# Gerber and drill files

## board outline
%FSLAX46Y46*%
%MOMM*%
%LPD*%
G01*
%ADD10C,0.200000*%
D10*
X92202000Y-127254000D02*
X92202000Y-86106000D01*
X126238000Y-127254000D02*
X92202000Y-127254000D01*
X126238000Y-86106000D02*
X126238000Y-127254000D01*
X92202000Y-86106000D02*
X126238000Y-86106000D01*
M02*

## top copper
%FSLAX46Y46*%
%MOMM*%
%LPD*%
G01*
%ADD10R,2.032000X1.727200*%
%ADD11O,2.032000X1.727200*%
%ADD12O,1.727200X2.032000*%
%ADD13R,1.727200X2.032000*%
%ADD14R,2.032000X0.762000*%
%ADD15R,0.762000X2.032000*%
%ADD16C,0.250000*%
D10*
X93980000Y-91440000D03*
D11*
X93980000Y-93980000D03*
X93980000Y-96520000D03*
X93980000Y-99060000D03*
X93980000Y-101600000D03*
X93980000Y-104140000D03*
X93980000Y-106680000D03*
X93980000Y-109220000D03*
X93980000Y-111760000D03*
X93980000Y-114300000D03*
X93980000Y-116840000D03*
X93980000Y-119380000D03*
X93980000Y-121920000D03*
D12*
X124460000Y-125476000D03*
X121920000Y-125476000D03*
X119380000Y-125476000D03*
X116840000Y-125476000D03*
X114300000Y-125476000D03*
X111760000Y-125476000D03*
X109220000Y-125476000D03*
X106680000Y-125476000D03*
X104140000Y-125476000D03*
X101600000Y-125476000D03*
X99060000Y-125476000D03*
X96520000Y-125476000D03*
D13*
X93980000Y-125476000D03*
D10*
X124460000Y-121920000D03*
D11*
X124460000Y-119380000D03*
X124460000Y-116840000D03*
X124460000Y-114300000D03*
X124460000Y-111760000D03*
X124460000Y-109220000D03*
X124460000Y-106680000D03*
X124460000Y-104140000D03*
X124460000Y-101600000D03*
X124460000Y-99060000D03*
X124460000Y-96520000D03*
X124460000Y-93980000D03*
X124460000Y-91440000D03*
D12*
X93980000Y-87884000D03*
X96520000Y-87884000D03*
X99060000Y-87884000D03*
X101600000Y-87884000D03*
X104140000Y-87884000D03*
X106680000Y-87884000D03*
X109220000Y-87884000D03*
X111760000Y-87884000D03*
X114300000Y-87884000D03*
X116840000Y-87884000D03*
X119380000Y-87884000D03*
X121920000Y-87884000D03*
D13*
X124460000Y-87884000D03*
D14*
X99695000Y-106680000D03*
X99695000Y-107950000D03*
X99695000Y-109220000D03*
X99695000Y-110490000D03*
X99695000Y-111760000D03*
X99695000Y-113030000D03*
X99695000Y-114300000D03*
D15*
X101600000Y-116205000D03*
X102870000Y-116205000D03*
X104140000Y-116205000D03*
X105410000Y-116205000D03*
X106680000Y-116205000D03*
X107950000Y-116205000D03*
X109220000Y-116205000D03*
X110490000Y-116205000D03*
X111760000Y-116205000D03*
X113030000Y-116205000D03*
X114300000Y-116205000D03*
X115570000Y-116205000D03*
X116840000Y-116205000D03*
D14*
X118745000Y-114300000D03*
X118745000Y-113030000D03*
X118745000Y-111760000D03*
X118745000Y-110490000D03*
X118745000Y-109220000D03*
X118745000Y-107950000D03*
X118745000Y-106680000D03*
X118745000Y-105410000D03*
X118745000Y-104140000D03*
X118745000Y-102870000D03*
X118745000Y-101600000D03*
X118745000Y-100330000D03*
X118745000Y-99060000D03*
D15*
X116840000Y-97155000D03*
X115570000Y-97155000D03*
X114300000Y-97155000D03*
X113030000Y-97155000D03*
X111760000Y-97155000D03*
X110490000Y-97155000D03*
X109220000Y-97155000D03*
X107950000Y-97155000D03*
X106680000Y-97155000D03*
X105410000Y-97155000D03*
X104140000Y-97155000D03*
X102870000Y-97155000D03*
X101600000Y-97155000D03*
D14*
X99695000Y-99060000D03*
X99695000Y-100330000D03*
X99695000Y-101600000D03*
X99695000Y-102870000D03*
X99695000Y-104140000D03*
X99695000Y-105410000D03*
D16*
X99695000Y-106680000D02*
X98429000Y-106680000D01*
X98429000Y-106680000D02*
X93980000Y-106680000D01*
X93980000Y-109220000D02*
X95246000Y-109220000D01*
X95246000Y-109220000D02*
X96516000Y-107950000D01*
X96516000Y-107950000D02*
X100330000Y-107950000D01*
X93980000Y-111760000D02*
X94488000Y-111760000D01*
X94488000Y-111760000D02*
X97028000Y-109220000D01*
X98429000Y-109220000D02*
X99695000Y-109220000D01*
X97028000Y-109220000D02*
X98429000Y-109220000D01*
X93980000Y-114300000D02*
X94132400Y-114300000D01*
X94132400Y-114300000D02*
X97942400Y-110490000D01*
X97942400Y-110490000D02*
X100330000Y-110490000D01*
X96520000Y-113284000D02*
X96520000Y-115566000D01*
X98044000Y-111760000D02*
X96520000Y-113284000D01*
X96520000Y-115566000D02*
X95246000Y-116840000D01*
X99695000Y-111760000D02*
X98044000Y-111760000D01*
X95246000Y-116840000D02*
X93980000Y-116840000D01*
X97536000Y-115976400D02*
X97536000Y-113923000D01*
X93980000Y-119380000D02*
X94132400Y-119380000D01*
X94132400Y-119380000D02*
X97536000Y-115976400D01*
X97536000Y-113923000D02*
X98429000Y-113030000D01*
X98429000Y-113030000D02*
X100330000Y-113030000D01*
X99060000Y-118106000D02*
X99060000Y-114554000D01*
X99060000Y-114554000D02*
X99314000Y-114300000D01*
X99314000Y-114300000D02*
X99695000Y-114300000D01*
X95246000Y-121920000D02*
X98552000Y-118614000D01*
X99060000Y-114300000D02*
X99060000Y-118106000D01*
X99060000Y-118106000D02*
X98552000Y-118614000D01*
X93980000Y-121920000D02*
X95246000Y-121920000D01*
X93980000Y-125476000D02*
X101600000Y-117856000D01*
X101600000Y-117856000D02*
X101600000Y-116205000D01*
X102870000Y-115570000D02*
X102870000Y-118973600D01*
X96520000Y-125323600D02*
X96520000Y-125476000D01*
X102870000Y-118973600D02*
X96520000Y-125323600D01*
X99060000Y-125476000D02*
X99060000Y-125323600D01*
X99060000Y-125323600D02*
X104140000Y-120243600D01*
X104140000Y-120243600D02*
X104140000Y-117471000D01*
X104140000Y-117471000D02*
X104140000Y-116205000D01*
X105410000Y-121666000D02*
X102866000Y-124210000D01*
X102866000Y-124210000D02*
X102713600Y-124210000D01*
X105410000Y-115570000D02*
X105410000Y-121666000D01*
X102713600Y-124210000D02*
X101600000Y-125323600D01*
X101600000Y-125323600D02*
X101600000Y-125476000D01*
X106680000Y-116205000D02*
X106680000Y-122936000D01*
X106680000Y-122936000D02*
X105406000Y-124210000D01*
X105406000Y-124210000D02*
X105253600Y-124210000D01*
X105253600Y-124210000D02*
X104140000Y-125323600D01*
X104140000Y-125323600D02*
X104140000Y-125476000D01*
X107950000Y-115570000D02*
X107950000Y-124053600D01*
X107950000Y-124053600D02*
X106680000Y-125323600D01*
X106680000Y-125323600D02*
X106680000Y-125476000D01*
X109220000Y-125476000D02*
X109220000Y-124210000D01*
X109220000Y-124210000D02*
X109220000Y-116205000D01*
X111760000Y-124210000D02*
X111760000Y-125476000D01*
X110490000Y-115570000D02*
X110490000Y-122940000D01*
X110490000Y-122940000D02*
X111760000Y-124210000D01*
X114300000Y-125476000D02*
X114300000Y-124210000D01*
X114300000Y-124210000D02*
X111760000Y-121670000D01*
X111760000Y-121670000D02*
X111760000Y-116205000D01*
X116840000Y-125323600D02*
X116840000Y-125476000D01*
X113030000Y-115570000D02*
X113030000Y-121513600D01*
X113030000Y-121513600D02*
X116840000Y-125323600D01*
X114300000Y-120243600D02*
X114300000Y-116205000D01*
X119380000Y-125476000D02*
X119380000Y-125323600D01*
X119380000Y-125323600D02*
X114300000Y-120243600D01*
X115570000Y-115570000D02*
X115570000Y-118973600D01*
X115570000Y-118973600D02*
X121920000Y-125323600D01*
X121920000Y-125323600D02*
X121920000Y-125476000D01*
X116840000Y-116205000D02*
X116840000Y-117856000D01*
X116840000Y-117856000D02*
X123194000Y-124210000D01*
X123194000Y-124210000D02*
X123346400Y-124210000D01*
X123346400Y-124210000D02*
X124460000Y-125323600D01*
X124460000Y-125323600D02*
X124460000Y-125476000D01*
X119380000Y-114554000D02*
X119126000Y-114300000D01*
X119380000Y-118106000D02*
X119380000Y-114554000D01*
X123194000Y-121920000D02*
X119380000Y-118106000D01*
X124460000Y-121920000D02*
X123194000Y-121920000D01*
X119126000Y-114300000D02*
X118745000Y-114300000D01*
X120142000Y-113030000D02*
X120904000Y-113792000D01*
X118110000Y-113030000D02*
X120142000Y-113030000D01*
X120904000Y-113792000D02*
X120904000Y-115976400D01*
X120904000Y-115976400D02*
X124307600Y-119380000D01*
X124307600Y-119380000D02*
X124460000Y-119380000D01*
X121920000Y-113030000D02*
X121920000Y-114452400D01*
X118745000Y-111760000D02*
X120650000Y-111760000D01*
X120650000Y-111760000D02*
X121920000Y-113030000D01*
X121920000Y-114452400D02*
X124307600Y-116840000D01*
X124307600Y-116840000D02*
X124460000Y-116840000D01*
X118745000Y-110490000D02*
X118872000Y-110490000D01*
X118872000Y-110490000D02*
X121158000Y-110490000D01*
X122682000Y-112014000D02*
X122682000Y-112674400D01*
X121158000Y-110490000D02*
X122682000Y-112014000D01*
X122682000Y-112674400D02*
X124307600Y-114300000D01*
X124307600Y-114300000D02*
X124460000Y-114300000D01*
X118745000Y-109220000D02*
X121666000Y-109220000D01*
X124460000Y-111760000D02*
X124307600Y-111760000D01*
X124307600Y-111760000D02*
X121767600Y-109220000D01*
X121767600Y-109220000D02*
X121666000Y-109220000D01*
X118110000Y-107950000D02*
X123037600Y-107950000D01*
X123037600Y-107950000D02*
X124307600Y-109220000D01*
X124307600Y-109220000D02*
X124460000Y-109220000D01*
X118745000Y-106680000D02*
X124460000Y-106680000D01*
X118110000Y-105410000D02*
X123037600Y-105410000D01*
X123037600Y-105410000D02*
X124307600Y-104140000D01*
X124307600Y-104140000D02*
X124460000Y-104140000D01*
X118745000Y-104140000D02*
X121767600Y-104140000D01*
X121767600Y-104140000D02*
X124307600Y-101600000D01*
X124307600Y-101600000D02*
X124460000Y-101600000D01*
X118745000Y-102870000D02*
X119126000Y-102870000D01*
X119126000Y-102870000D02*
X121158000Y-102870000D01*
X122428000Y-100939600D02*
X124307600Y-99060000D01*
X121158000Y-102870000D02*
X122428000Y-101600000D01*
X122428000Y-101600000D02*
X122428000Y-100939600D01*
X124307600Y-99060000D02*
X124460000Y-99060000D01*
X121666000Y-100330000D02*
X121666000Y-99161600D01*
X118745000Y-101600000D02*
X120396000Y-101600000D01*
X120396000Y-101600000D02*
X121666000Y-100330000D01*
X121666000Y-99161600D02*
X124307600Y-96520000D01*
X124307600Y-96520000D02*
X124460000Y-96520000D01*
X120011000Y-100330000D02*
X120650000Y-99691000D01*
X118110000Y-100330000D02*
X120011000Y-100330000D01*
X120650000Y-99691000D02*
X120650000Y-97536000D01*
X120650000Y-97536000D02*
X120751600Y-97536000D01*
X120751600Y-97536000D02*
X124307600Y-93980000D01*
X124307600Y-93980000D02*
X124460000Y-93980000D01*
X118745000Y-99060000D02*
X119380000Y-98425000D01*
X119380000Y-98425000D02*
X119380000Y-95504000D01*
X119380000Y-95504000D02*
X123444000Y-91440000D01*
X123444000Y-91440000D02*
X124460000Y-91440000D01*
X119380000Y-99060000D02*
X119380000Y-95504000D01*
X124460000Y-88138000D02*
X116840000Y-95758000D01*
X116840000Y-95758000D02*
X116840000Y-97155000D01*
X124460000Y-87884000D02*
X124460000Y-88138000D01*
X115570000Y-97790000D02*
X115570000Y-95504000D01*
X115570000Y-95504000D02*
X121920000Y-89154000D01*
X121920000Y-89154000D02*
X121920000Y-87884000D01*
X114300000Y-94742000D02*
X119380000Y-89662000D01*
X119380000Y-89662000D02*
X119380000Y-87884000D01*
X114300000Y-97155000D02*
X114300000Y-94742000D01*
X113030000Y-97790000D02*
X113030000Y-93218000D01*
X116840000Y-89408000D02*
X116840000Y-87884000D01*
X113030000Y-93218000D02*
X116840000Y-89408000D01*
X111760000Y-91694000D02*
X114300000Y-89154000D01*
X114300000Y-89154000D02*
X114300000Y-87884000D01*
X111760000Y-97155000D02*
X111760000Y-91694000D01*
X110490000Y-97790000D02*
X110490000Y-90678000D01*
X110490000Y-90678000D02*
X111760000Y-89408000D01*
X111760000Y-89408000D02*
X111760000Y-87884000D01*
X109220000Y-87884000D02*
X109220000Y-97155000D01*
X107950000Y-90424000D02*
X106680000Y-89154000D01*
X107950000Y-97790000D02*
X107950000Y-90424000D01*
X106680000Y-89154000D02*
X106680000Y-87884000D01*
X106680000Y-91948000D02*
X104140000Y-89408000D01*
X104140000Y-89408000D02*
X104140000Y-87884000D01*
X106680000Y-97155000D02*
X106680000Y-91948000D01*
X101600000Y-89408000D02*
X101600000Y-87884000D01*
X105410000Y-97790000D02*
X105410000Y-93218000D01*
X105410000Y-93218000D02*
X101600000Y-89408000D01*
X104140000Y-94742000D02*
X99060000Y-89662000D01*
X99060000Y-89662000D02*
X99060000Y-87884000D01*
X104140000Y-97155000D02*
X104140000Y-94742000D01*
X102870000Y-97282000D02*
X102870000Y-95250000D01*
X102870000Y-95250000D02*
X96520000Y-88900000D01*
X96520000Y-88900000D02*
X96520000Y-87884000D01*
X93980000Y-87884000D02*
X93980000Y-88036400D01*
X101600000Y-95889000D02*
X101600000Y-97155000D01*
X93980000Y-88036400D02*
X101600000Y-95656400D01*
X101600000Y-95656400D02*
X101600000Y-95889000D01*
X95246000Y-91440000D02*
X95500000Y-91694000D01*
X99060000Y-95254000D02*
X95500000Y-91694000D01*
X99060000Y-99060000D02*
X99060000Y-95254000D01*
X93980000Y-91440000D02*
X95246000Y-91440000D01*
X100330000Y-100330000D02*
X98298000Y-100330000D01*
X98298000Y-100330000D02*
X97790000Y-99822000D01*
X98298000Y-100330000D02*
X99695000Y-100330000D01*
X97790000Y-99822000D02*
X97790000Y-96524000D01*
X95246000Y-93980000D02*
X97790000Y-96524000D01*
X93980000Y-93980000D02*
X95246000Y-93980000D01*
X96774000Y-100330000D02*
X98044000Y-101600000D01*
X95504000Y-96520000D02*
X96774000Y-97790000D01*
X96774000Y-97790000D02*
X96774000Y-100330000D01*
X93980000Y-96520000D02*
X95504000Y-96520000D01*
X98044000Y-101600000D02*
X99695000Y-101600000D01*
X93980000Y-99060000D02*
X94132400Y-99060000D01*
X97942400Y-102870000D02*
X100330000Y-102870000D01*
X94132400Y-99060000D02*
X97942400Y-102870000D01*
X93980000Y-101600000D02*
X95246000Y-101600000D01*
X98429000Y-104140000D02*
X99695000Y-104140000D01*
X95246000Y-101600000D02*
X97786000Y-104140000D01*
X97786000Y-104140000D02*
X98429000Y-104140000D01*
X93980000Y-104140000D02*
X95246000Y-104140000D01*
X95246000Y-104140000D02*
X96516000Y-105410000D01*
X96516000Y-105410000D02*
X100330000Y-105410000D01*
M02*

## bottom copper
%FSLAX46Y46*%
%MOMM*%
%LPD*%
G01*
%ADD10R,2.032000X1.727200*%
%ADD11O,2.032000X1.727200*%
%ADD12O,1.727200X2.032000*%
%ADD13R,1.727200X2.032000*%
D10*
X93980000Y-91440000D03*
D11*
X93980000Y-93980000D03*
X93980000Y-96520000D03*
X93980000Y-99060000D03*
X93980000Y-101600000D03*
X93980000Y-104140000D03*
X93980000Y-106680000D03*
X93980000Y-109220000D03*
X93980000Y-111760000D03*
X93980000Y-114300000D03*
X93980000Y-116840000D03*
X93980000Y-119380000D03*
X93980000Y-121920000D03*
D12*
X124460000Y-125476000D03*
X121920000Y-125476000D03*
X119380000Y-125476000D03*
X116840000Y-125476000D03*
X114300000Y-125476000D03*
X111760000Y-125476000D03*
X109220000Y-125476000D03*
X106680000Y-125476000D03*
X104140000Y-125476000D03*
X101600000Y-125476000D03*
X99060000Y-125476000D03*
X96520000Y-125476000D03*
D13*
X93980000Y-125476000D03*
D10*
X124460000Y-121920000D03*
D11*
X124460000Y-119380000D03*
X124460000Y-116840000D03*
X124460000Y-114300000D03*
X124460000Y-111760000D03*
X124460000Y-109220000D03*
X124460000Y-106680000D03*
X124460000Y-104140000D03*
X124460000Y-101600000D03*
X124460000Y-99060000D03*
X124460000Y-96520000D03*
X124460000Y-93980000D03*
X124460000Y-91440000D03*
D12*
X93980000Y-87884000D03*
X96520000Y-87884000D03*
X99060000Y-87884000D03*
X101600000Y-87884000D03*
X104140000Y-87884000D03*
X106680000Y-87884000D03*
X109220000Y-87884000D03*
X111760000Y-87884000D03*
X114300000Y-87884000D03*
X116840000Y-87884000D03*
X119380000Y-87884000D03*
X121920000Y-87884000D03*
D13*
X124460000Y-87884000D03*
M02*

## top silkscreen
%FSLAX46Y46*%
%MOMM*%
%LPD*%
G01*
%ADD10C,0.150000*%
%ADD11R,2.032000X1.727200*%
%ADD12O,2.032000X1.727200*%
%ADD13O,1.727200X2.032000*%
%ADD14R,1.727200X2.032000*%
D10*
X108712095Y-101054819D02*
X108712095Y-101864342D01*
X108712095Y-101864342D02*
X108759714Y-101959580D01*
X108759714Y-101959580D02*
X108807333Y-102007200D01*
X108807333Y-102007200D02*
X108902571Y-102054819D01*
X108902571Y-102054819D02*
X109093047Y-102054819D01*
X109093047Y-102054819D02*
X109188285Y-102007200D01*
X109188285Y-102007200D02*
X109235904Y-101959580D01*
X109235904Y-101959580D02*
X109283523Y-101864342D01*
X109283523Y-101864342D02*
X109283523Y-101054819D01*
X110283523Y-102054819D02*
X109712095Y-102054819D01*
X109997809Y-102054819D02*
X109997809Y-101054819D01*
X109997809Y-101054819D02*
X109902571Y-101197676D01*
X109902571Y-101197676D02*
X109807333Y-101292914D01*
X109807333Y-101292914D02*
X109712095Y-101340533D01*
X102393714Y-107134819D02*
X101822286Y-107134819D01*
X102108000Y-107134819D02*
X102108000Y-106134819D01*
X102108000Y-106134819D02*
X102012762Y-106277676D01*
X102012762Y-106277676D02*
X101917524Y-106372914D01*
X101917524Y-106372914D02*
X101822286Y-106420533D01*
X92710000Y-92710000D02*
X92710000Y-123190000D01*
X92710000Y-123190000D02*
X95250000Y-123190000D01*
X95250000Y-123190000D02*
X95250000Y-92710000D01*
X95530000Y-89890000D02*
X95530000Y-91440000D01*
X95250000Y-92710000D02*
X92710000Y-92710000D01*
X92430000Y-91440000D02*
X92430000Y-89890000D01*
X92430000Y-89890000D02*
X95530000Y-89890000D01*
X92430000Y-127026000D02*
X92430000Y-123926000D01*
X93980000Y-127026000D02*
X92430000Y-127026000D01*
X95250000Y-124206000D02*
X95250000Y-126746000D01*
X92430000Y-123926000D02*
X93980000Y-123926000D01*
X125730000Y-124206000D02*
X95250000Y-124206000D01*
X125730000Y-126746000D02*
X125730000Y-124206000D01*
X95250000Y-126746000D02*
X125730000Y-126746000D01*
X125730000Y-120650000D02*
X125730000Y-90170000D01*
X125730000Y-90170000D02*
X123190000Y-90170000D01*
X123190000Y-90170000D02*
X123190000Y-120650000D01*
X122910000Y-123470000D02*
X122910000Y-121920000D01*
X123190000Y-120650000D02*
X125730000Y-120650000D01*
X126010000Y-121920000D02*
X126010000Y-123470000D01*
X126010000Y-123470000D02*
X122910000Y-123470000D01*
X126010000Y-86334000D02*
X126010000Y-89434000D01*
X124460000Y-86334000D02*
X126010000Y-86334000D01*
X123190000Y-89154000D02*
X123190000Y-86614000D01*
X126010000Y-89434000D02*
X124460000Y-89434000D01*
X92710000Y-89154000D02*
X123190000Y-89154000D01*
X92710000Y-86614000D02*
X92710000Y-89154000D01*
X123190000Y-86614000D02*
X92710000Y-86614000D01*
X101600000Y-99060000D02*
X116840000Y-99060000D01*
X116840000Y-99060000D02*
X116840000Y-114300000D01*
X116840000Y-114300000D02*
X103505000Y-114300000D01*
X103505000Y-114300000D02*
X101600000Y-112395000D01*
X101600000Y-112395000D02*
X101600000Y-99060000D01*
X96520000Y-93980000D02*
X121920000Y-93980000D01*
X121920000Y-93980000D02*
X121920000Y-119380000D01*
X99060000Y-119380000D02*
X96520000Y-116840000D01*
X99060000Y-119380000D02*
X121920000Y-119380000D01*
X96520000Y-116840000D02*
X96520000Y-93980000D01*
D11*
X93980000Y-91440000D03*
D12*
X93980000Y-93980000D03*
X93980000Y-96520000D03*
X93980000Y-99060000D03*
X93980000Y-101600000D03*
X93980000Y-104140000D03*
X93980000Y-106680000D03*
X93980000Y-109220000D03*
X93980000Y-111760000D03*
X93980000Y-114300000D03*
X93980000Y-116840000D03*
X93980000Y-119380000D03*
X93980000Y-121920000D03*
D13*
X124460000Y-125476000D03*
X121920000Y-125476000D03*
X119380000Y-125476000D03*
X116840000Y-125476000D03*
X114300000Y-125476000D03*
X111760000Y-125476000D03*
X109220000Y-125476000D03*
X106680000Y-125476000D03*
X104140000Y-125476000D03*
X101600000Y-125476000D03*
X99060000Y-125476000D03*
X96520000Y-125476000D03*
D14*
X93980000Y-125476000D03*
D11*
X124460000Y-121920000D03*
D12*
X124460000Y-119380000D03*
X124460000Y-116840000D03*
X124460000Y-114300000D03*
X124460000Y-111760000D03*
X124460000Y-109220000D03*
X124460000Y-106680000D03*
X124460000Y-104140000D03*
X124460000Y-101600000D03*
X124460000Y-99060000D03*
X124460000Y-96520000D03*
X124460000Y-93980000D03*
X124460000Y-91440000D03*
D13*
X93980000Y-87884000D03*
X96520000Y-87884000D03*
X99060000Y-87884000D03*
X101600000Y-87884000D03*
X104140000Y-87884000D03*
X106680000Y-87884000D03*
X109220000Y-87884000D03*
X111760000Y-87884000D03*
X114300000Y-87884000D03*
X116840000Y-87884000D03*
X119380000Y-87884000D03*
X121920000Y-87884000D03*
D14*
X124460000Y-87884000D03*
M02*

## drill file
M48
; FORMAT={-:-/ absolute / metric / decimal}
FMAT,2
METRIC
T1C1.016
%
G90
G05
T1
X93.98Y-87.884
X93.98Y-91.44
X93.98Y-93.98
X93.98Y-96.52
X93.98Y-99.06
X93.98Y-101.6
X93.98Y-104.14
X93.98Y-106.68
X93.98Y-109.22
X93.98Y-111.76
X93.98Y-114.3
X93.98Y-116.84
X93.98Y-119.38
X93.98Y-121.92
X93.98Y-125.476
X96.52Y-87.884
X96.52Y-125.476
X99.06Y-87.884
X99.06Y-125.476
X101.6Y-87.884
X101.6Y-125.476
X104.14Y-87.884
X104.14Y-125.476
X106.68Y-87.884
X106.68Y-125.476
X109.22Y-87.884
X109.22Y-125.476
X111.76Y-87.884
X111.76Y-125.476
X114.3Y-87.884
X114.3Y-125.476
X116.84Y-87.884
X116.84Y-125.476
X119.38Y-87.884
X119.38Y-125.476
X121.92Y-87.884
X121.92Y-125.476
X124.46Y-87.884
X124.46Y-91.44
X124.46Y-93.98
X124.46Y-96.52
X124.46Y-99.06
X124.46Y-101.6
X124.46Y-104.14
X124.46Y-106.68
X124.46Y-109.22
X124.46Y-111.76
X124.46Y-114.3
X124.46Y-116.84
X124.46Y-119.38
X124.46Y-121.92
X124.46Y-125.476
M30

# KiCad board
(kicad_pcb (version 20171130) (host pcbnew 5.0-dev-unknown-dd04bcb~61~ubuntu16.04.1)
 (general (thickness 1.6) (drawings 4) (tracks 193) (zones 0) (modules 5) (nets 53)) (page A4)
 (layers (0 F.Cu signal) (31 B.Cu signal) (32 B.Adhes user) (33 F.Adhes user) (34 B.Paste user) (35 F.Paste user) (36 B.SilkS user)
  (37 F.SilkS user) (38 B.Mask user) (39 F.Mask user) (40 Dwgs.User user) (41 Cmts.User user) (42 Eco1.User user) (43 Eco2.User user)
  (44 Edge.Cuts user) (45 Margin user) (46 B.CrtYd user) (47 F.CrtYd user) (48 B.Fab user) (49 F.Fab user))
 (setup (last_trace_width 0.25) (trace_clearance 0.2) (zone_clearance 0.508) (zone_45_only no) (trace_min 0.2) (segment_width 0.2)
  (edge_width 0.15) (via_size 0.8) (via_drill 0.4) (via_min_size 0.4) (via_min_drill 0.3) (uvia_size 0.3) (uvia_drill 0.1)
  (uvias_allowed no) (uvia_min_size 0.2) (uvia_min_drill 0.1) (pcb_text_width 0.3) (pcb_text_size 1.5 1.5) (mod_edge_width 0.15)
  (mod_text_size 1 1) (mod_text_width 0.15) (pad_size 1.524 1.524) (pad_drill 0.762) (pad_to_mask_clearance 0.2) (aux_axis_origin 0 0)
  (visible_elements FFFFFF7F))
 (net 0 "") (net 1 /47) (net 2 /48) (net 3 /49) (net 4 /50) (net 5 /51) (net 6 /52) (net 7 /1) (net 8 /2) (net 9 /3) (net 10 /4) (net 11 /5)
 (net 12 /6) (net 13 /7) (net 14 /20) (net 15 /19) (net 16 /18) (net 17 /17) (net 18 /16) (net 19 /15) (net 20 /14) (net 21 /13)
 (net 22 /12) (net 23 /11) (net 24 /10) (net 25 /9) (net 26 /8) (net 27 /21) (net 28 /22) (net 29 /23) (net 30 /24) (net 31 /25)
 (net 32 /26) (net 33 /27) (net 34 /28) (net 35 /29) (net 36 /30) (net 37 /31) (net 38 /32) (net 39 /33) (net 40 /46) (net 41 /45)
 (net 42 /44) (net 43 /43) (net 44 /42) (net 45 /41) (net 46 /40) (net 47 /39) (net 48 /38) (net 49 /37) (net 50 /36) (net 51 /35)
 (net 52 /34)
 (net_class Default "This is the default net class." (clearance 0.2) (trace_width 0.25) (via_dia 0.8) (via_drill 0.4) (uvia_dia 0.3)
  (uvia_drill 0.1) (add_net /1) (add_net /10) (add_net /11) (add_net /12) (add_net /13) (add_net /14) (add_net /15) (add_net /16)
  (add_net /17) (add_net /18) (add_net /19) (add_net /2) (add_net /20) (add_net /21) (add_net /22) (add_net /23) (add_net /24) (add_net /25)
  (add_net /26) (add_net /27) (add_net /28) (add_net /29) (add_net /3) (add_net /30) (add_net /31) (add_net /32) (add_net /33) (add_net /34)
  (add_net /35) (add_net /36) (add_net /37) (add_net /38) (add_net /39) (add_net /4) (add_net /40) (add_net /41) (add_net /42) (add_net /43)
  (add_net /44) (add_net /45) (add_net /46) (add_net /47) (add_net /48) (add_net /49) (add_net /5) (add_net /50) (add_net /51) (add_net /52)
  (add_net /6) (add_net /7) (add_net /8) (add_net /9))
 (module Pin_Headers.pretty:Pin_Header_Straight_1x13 (layer F.Cu) (at 93.98 91.44)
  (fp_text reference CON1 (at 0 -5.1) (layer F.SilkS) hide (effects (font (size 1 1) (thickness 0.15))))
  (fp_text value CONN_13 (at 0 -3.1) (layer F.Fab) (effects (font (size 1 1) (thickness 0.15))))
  (fp_line (start -1.27 1.27) (end -1.27 31.75) (layer F.SilkS) (width 0.15))
  (fp_line (start -1.27 31.75) (end 1.27 31.75) (layer F.SilkS) (width 0.15))
  (fp_line (start 1.27 31.75) (end 1.27 1.27) (layer F.SilkS) (width 0.15))
  (fp_line (start 1.55 -1.55) (end 1.55 0) (layer F.SilkS) (width 0.15))
  (fp_line (start 1.27 1.27) (end -1.27 1.27) (layer F.SilkS) (width 0.15))
  (fp_line (start -1.55 0) (end -1.55 -1.55) (layer F.SilkS) (width 0.15))
  (fp_line (start -1.55 -1.55) (end 1.55 -1.55) (layer F.SilkS) (width 0.15))
  (pad 1 thru_hole rect (at 0 0) (size 2.032 1.7272) (drill 1.016) (layers *.Cu *.Mask F.SilkS) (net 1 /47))
  (pad 2 thru_hole oval (at 0 2.54) (size 2.032 1.7272) (drill 1.016) (layers *.Cu *.Mask F.SilkS) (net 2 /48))
  (pad 3 thru_hole oval (at 0 5.08) (size 2.032 1.7272) (drill 1.016) (layers *.Cu *.Mask F.SilkS) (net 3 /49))
  (pad 4 thru_hole oval (at 0 7.62) (size 2.032 1.7272) (drill 1.016) (layers *.Cu *.Mask F.SilkS) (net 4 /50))
  (pad 5 thru_hole oval (at 0 10.16) (size 2.032 1.7272) (drill 1.016) (layers *.Cu *.Mask F.SilkS) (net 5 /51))
  (pad 6 thru_hole oval (at 0 12.7) (size 2.032 1.7272) (drill 1.016) (layers *.Cu *.Mask F.SilkS) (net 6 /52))
  (pad 7 thru_hole oval (at 0 15.24) (size 2.032 1.7272) (drill 1.016) (layers *.Cu *.Mask F.SilkS) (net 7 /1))
  (pad 8 thru_hole oval (at 0 17.78) (size 2.032 1.7272) (drill 1.016) (layers *.Cu *.Mask F.SilkS) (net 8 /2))
  (pad 9 thru_hole oval (at 0 20.32) (size 2.032 1.7272) (drill 1.016) (layers *.Cu *.Mask F.SilkS) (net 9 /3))
  (pad 10 thru_hole oval (at 0 22.86) (size 2.032 1.7272) (drill 1.016) (layers *.Cu *.Mask F.SilkS) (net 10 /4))
  (pad 11 thru_hole oval (at 0 25.4) (size 2.032 1.7272) (drill 1.016) (layers *.Cu *.Mask F.SilkS) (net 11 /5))
  (pad 12 thru_hole oval (at 0 27.94) (size 2.032 1.7272) (drill 1.016) (layers *.Cu *.Mask F.SilkS) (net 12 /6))
  (pad 13 thru_hole oval (at 0 30.48) (size 2.032 1.7272) (drill 1.016) (layers *.Cu *.Mask F.SilkS) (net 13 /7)))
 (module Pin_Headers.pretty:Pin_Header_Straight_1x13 (layer F.Cu) (at 93.98 125.476 90)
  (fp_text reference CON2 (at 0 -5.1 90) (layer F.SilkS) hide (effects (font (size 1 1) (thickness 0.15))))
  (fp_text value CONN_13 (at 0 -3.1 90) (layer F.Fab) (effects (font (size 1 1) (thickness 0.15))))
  (fp_line (start -1.55 -1.55) (end 1.55 -1.55) (layer F.SilkS) (width 0.15))
  (fp_line (start -1.55 0) (end -1.55 -1.55) (layer F.SilkS) (width 0.15))
  (fp_line (start 1.27 1.27) (end -1.27 1.27) (layer F.SilkS) (width 0.15))
  (fp_line (start 1.55 -1.55) (end 1.55 0) (layer F.SilkS) (width 0.15))
  (fp_line (start 1.27 31.75) (end 1.27 1.27) (layer F.SilkS) (width 0.15))
  (fp_line (start -1.27 31.75) (end 1.27 31.75) (layer F.SilkS) (width 0.15))
  (fp_line (start -1.27 1.27) (end -1.27 31.75) (layer F.SilkS) (width 0.15))
  (pad 13 thru_hole oval (at 0 30.48 90) (size 2.032 1.7272) (drill 1.016) (layers *.Cu *.Mask F.SilkS) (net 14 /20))
  (pad 12 thru_hole oval (at 0 27.94 90) (size 2.032 1.7272) (drill 1.016) (layers *.Cu *.Mask F.SilkS) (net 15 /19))
  (pad 11 thru_hole oval (at 0 25.4 90) (size 2.032 1.7272) (drill 1.016) (layers *.Cu *.Mask F.SilkS) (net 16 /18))
  (pad 10 thru_hole oval (at 0 22.86 90) (size 2.032 1.7272) (drill 1.016) (layers *.Cu *.Mask F.SilkS) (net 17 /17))
  (pad 9 thru_hole oval (at 0 20.32 90) (size 2.032 1.7272) (drill 1.016) (layers *.Cu *.Mask F.SilkS) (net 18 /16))
  (pad 8 thru_hole oval (at 0 17.78 90) (size 2.032 1.7272) (drill 1.016) (layers *.Cu *.Mask F.SilkS) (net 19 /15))
  (pad 7 thru_hole oval (at 0 15.24 90) (size 2.032 1.7272) (drill 1.016) (layers *.Cu *.Mask F.SilkS) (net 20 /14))
  (pad 6 thru_hole oval (at 0 12.7 90) (size 2.032 1.7272) (drill 1.016) (layers *.Cu *.Mask F.SilkS) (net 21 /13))
  (pad 5 thru_hole oval (at 0 10.16 90) (size 2.032 1.7272) (drill 1.016) (layers *.Cu *.Mask F.SilkS) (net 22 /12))
  (pad 4 thru_hole oval (at 0 7.62 90) (size 2.032 1.7272) (drill 1.016) (layers *.Cu *.Mask F.SilkS) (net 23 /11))
  (pad 3 thru_hole oval (at 0 5.08 90) (size 2.032 1.7272) (drill 1.016) (layers *.Cu *.Mask F.SilkS) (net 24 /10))
  (pad 2 thru_hole oval (at 0 2.54 90) (size 2.032 1.7272) (drill 1.016) (layers *.Cu *.Mask F.SilkS) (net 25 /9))
  (pad 1 thru_hole rect (at 0 0 90) (size 2.032 1.7272) (drill 1.016) (layers *.Cu *.Mask F.SilkS) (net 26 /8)))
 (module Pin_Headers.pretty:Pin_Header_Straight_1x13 (layer F.Cu) (at 124.46 121.92 180)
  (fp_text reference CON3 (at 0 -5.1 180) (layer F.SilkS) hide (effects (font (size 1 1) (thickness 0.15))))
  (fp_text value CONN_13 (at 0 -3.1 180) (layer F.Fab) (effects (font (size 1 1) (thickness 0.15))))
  (fp_line (start -1.27 1.27) (end -1.27 31.75) (layer F.SilkS) (width 0.15))
  (fp_line (start -1.27 31.75) (end 1.27 31.75) (layer F.SilkS) (width 0.15))
  (fp_line (start 1.27 31.75) (end 1.27 1.27) (layer F.SilkS) (width 0.15))
  (fp_line (start 1.55 -1.55) (end 1.55 0) (layer F.SilkS) (width 0.15))
  (fp_line (start 1.27 1.27) (end -1.27 1.27) (layer F.SilkS) (width 0.15))
  (fp_line (start -1.55 0) (end -1.55 -1.55) (layer F.SilkS) (width 0.15))
  (fp_line (start -1.55 -1.55) (end 1.55 -1.55) (layer F.SilkS) (width 0.15))
  (pad 1 thru_hole rect (at 0 0 180) (size 2.032 1.7272) (drill 1.016) (layers *.Cu *.Mask F.SilkS) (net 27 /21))
  (pad 2 thru_hole oval (at 0 2.54 180) (size 2.032 1.7272) (drill 1.016) (layers *.Cu *.Mask F.SilkS) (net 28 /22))
  (pad 3 thru_hole oval (at 0 5.08 180) (size 2.032 1.7272) (drill 1.016) (layers *.Cu *.Mask F.SilkS) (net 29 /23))
  (pad 4 thru_hole oval (at 0 7.62 180) (size 2.032 1.7272) (drill 1.016) (layers *.Cu *.Mask F.SilkS) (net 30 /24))
  (pad 5 thru_hole oval (at 0 10.16 180) (size 2.032 1.7272) (drill 1.016) (layers *.Cu *.Mask F.SilkS) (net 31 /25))
  (pad 6 thru_hole oval (at 0 12.7 180) (size 2.032 1.7272) (drill 1.016) (layers *.Cu *.Mask F.SilkS) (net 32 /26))
  (pad 7 thru_hole oval (at 0 15.24 180) (size 2.032 1.7272) (drill 1.016) (layers *.Cu *.Mask F.SilkS) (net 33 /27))
  (pad 8 thru_hole oval (at 0 17.78 180) (size 2.032 1.7272) (drill 1.016) (layers *.Cu *.Mask F.SilkS) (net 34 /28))
  (pad 9 thru_hole oval (at 0 20.32 180) (size 2.032 1.7272) (drill 1.016) (layers *.Cu *.Mask F.SilkS) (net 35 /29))
  (pad 10 thru_hole oval (at 0 22.86 180) (size 2.032 1.7272) (drill 1.016) (layers *.Cu *.Mask F.SilkS) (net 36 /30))
  (pad 11 thru_hole oval (at 0 25.4 180) (size 2.032 1.7272) (drill 1.016) (layers *.Cu *.Mask F.SilkS) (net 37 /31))
  (pad 12 thru_hole oval (at 0 27.94 180) (size 2.032 1.7272) (drill 1.016) (layers *.Cu *.Mask F.SilkS) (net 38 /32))
  (pad 13 thru_hole oval (at 0 30.48 180) (size 2.032 1.7272) (drill 1.016) (layers *.Cu *.Mask F.SilkS) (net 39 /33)))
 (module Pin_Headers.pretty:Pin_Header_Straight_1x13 (layer F.Cu) (at 124.46 87.884 270)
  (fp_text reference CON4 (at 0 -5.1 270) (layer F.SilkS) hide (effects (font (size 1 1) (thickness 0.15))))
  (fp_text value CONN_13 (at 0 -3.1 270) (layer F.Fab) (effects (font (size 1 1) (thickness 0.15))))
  (fp_line (start -1.55 -1.55) (end 1.55 -1.55) (layer F.SilkS) (width 0.15))
  (fp_line (start -1.55 0) (end -1.55 -1.55) (layer F.SilkS) (width 0.15))
  (fp_line (start 1.27 1.27) (end -1.27 1.27) (layer F.SilkS) (width 0.15))
  (fp_line (start 1.55 -1.55) (end 1.55 0) (layer F.SilkS) (width 0.15))
  (fp_line (start 1.27 31.75) (end 1.27 1.27) (layer F.SilkS) (width 0.15))
  (fp_line (start -1.27 31.75) (end 1.27 31.75) (layer F.SilkS) (width 0.15))
  (fp_line (start -1.27 1.27) (end -1.27 31.75) (layer F.SilkS) (width 0.15))
  (pad 13 thru_hole oval (at 0 30.48 270) (size 2.032 1.7272) (drill 1.016) (layers *.Cu *.Mask F.SilkS) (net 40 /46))
  (pad 12 thru_hole oval (at 0 27.94 270) (size 2.032 1.7272) (drill 1.016) (layers *.Cu *.Mask F.SilkS) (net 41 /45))
  (pad 11 thru_hole oval (at 0 25.4 270) (size 2.032 1.7272) (drill 1.016) (layers *.Cu *.Mask F.SilkS) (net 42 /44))
  (pad 10 thru_hole oval (at 0 22.86 270) (size 2.032 1.7272) (drill 1.016) (layers *.Cu *.Mask F.SilkS) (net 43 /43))
  (pad 9 thru_hole oval (at 0 20.32 270) (size 2.032 1.7272) (drill 1.016) (layers *.Cu *.Mask F.SilkS) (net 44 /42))
  (pad 8 thru_hole oval (at 0 17.78 270) (size 2.032 1.7272) (drill 1.016) (layers *.Cu *.Mask F.SilkS) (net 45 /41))
  (pad 7 thru_hole oval (at 0 15.24 270) (size 2.032 1.7272) (drill 1.016) (layers *.Cu *.Mask F.SilkS) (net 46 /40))
  (pad 6 thru_hole oval (at 0 12.7 270) (size 2.032 1.7272) (drill 1.016) (layers *.Cu *.Mask F.SilkS) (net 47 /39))
  (pad 5 thru_hole oval (at 0 10.16 270) (size 2.032 1.7272) (drill 1.016) (layers *.Cu *.Mask F.SilkS) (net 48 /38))
  (pad 4 thru_hole oval (at 0 7.62 270) (size 2.032 1.7272) (drill 1.016) (layers *.Cu *.Mask F.SilkS) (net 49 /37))
  (pad 3 thru_hole oval (at 0 5.08 270) (size 2.032 1.7272) (drill 1.016) (layers *.Cu *.Mask F.SilkS) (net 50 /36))
  (pad 2 thru_hole oval (at 0 2.54 270) (size 2.032 1.7272) (drill 1.016) (layers *.Cu *.Mask F.SilkS) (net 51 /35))
  (pad 1 thru_hole rect (at 0 0 270) (size 2.032 1.7272) (drill 1.016) (layers *.Cu *.Mask F.SilkS) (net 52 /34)))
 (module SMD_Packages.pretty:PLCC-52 (layer F.Cu) (at 109.22 106.68)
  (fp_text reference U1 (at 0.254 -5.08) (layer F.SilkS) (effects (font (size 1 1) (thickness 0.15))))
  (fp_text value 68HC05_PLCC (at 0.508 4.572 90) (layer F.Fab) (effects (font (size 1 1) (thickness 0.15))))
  (fp_line (start -7.62 -7.62) (end 7.62 -7.62) (layer F.SilkS) (width 0.15))
  (fp_line (start 7.62 -7.62) (end 7.62 7.62) (layer F.SilkS) (width 0.15))
  (fp_line (start 7.62 7.62) (end -5.715 7.62) (layer F.SilkS) (width 0.15))
  (fp_line (start -5.715 7.62) (end -7.62 5.715) (layer F.SilkS) (width 0.15))
  (fp_line (start -7.62 5.715) (end -7.62 -7.62) (layer F.SilkS) (width 0.15))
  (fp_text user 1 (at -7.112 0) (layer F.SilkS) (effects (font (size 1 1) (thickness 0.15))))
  (fp_line (start -12.7 -12.7) (end 12.7 -12.7) (layer F.SilkS) (width 0.15))
  (fp_line (start 12.7 -12.7) (end 12.7 12.7) (layer F.SilkS) (width 0.15))
  (fp_line (start -10.16 12.7) (end -12.7 10.16) (layer F.SilkS) (width 0.15))
  (fp_line (start -10.16 12.7) (end 12.7 12.7) (layer F.SilkS) (width 0.15))
  (fp_line (start -12.7 10.16) (end -12.7 -12.7) (layer F.SilkS) (width 0.15))
  (pad 1 smd rect (at -9.525 0) (size 2.032 0.762) (layers F.Cu F.Paste F.Mask) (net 7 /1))
  (pad 2 smd rect (at -9.525 1.27) (size 2.032 0.762) (layers F.Cu F.Paste F.Mask) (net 8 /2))
  (pad 3 smd rect (at -9.525 2.54) (size 2.032 0.762) (layers F.Cu F.Paste F.Mask) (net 9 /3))
  (pad 4 smd rect (at -9.525 3.81) (size 2.032 0.762) (layers F.Cu F.Paste F.Mask) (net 10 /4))
  (pad 5 smd rect (at -9.525 5.08) (size 2.032 0.762) (layers F.Cu F.Paste F.Mask) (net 11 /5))
  (pad 6 smd rect (at -9.525 6.35) (size 2.032 0.762) (layers F.Cu F.Paste F.Mask) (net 12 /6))
  (pad 7 smd rect (at -9.525 7.62) (size 2.032 0.762) (layers F.Cu F.Paste F.Mask) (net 13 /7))
  (pad 8 smd rect (at -7.62 9.525) (size 0.762 2.032) (layers F.Cu F.Paste F.Mask) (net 26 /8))
  (pad 9 smd rect (at -6.35 9.525) (size 0.762 2.032) (layers F.Cu F.Paste F.Mask) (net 25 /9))
  (pad 10 smd rect (at -5.08 9.525) (size 0.762 2.032) (layers F.Cu F.Paste F.Mask) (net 24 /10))
  (pad 11 smd rect (at -3.81 9.525) (size 0.762 2.032) (layers F.Cu F.Paste F.Mask) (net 23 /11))
  (pad 12 smd rect (at -2.54 9.525) (size 0.762 2.032) (layers F.Cu F.Paste F.Mask) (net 22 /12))
  (pad 13 smd rect (at -1.27 9.525) (size 0.762 2.032) (layers F.Cu F.Paste F.Mask) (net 21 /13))
  (pad 14 smd rect (at 0 9.525) (size 0.762 2.032) (layers F.Cu F.Paste F.Mask) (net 20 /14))
  (pad 15 smd rect (at 1.27 9.525) (size 0.762 2.032) (layers F.Cu F.Paste F.Mask) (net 19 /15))
  (pad 16 smd rect (at 2.54 9.525) (size 0.762 2.032) (layers F.Cu F.Paste F.Mask) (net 18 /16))
  (pad 17 smd rect (at 3.81 9.525) (size 0.762 2.032) (layers F.Cu F.Paste F.Mask) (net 17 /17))
  (pad 18 smd rect (at 5.08 9.525) (size 0.762 2.032) (layers F.Cu F.Paste F.Mask) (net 16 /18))
  (pad 19 smd rect (at 6.35 9.525) (size 0.762 2.032) (layers F.Cu F.Paste F.Mask) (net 15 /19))
  (pad 20 smd rect (at 7.62 9.525) (size 0.762 2.032) (layers F.Cu F.Paste F.Mask) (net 14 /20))
  (pad 21 smd rect (at 9.525 7.62) (size 2.032 0.762) (layers F.Cu F.Paste F.Mask) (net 27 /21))
  (pad 22 smd rect (at 9.525 6.35) (size 2.032 0.762) (layers F.Cu F.Paste F.Mask) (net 28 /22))
  (pad 23 smd rect (at 9.525 5.08) (size 2.032 0.762) (layers F.Cu F.Paste F.Mask) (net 29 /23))
  (pad 24 smd rect (at 9.525 3.81) (size 2.032 0.762) (layers F.Cu F.Paste F.Mask) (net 30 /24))
  (pad 25 smd rect (at 9.525 2.54) (size 2.032 0.762) (layers F.Cu F.Paste F.Mask) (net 31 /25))
  (pad 26 smd rect (at 9.525 1.27) (size 2.032 0.762) (layers F.Cu F.Paste F.Mask) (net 32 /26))
  (pad 27 smd rect (at 9.525 0) (size 2.032 0.762) (layers F.Cu F.Paste F.Mask) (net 33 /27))
  (pad 28 smd rect (at 9.525 -1.27) (size 2.032 0.762) (layers F.Cu F.Paste F.Mask) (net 34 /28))
  (pad 29 smd rect (at 9.525 -2.54) (size 2.032 0.762) (layers F.Cu F.Paste F.Mask) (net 35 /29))
  (pad 30 smd rect (at 9.525 -3.81) (size 2.032 0.762) (layers F.Cu F.Paste F.Mask) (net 36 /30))
  (pad 31 smd rect (at 9.525 -5.08) (size 2.032 0.762) (layers F.Cu F.Paste F.Mask) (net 37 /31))
  (pad 32 smd rect (at 9.525 -6.35) (size 2.032 0.762) (layers F.Cu F.Paste F.Mask) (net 38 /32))
  (pad 33 smd rect (at 9.525 -7.62) (size 2.032 0.762) (layers F.Cu F.Paste F.Mask) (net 39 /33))
  (pad 34 smd rect (at 7.62 -9.525) (size 0.762 2.032) (layers F.Cu F.Paste F.Mask) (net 52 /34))
  (pad 35 smd rect (at 6.35 -9.525) (size 0.762 2.032) (layers F.Cu F.Paste F.Mask) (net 51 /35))
  (pad 36 smd rect (at 5.08 -9.525) (size 0.762 2.032) (layers F.Cu F.Paste F.Mask) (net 50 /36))
  (pad 37 smd rect (at 3.81 -9.525) (size 0.762 2.032) (layers F.Cu F.Paste F.Mask) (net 49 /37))
  (pad 38 smd rect (at 2.54 -9.525) (size 0.762 2.032) (layers F.Cu F.Paste F.Mask) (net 48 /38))
  (pad 39 smd rect (at 1.27 -9.525) (size 0.762 2.032) (layers F.Cu F.Paste F.Mask) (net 47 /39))
  (pad 40 smd rect (at 0 -9.525) (size 0.762 2.032) (layers F.Cu F.Paste F.Mask) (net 46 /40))
  (pad 41 smd rect (at -1.27 -9.525) (size 0.762 2.032) (layers F.Cu F.Paste F.Mask) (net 45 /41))
  (pad 42 smd rect (at -2.54 -9.525) (size 0.762 2.032) (layers F.Cu F.Paste F.Mask) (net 44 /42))
  (pad 43 smd rect (at -3.81 -9.525) (size 0.762 2.032) (layers F.Cu F.Paste F.Mask) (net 43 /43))
  (pad 44 smd rect (at -5.08 -9.525) (size 0.762 2.032) (layers F.Cu F.Paste F.Mask) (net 42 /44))
  (pad 45 smd rect (at -6.35 -9.525) (size 0.762 2.032) (layers F.Cu F.Paste F.Mask) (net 41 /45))
  (pad 46 smd rect (at -7.62 -9.525) (size 0.762 2.032) (layers F.Cu F.Paste F.Mask) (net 40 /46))
  (pad 47 smd rect (at -9.525 -7.62) (size 2.032 0.762) (layers F.Cu F.Paste F.Mask) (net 1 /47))
  (pad 48 smd rect (at -9.525 -6.35) (size 2.032 0.762) (layers F.Cu F.Paste F.Mask) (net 2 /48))
  (pad 49 smd rect (at -9.525 -5.08) (size 2.032 0.762) (layers F.Cu F.Paste F.Mask) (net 3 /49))
  (pad 50 smd rect (at -9.525 -3.81) (size 2.032 0.762) (layers F.Cu F.Paste F.Mask) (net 4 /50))
  (pad 51 smd rect (at -9.525 -2.54) (size 2.032 0.762) (layers F.Cu F.Paste F.Mask) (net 5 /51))
  (pad 52 smd rect (at -9.525 -1.27) (size 2.032 0.762) (layers F.Cu F.Paste F.Mask) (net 6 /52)))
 (gr_line (start 92.202 127.254) (end 92.202 86.106) (layer Edge.Cuts) (width 0.2))
 (gr_line (start 126.238 127.254) (end 92.202 127.254) (layer Edge.Cuts) (width 0.2))
 (gr_line (start 126.238 86.106) (end 126.238 127.254) (layer Edge.Cuts) (width 0.2))
 (gr_line (start 92.202 86.106) (end 126.238 86.106) (layer Edge.Cuts) (width 0.2))
 (segment (start 99.695 106.68) (end 98.429 106.68) (width 0.25) (layer F.Cu) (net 7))
 (segment (start 98.429 106.68) (end 93.98 106.68) (width 0.25) (layer F.Cu) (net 7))
 (segment (start 93.98 109.22) (end 95.246 109.22) (width 0.25) (layer F.Cu) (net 8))
 (segment (start 95.246 109.22) (end 96.516 107.95) (width 0.25) (layer F.Cu) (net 8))
 (segment (start 96.516 107.95) (end 100.33 107.95) (width 0.25) (layer F.Cu) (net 8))
 (segment (start 93.98 111.76) (end 94.488 111.76) (width 0.25) (layer F.Cu) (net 9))
 (segment (start 94.488 111.76) (end 97.028 109.22) (width 0.25) (layer F.Cu) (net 9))
 (segment (start 98.429 109.22) (end 99.695 109.22) (width 0.25) (layer F.Cu) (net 9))
 (segment (start 97.028 109.22) (end 98.429 109.22) (width 0.25) (layer F.Cu) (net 9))
 (segment (start 93.98 114.3) (end 94.1324 114.3) (width 0.25) (layer F.Cu) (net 10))
 (segment (start 94.1324 114.3) (end 97.9424 110.49) (width 0.25) (layer F.Cu) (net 10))
 (segment (start 97.9424 110.49) (end 100.33 110.49) (width 0.25) (layer F.Cu) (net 10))
 (segment (start 96.52 113.284) (end 96.52 115.566) (width 0.25) (layer F.Cu) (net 11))
 (segment (start 98.044 111.76) (end 96.52 113.284) (width 0.25) (layer F.Cu) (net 11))
 (segment (start 96.52 115.566) (end 95.246 116.84) (width 0.25) (layer F.Cu) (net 11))
 (segment (start 99.695 111.76) (end 98.044 111.76) (width 0.25) (layer F.Cu) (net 11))
 (segment (start 95.246 116.84) (end 93.98 116.84) (width 0.25) (layer F.Cu) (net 11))
 (segment (start 97.536 115.9764) (end 97.536 113.923) (width 0.25) (layer F.Cu) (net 12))
 (segment (start 93.98 119.38) (end 94.1324 119.38) (width 0.25) (layer F.Cu) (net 12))
 (segment (start 94.1324 119.38) (end 97.536 115.9764) (width 0.25) (layer F.Cu) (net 12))
 (segment (start 97.536 113.923) (end 98.429 113.03) (width 0.25) (layer F.Cu) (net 12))
 (segment (start 98.429 113.03) (end 100.33 113.03) (width 0.25) (layer F.Cu) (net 12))
 (segment (start 99.06 118.106) (end 99.06 114.554) (width 0.25) (layer F.Cu) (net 13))
 (segment (start 99.06 114.554) (end 99.314 114.3) (width 0.25) (layer F.Cu) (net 13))
 (segment (start 99.314 114.3) (end 99.695 114.3) (width 0.25) (layer F.Cu) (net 13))
 (segment (start 95.246 121.92) (end 98.552 118.614) (width 0.25) (layer F.Cu) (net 13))
 (segment (start 99.06 114.3) (end 99.06 118.106) (width 0.25) (layer F.Cu) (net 13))
 (segment (start 99.06 118.106) (end 98.552 118.614) (width 0.25) (layer F.Cu) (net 13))
 (segment (start 93.98 121.92) (end 95.246 121.92) (width 0.25) (layer F.Cu) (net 13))
 (segment (start 93.98 125.476) (end 101.6 117.856) (width 0.25) (layer F.Cu) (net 26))
 (segment (start 101.6 117.856) (end 101.6 116.205) (width 0.25) (layer F.Cu) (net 26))
 (segment (start 102.87 115.57) (end 102.87 118.9736) (width 0.25) (layer F.Cu) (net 25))
 (segment (start 96.52 125.3236) (end 96.52 125.476) (width 0.25) (layer F.Cu) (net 25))
 (segment (start 102.87 118.9736) (end 96.52 125.3236) (width 0.25) (layer F.Cu) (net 25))
 (segment (start 99.06 125.476) (end 99.06 125.3236) (width 0.25) (layer F.Cu) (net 24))
 (segment (start 99.06 125.3236) (end 104.14 120.2436) (width 0.25) (layer F.Cu) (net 24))
 (segment (start 104.14 120.2436) (end 104.14 117.471) (width 0.25) (layer F.Cu) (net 24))
 (segment (start 104.14 117.471) (end 104.14 116.205) (width 0.25) (layer F.Cu) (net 24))
 (segment (start 105.41 121.666) (end 102.866 124.21) (width 0.25) (layer F.Cu) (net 23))
 (segment (start 102.866 124.21) (end 102.7136 124.21) (width 0.25) (layer F.Cu) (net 23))
 (segment (start 105.41 115.57) (end 105.41 121.666) (width 0.25) (layer F.Cu) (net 23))
 (segment (start 102.7136 124.21) (end 101.6 125.3236) (width 0.25) (layer F.Cu) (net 23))
 (segment (start 101.6 125.3236) (end 101.6 125.476) (width 0.25) (layer F.Cu) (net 23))
 (segment (start 106.68 116.205) (end 106.68 122.936) (width 0.25) (layer F.Cu) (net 22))
 (segment (start 106.68 122.936) (end 105.406 124.21) (width 0.25) (layer F.Cu) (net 22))
 (segment (start 105.406 124.21) (end 105.2536 124.21) (width 0.25) (layer F.Cu) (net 22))
 (segment (start 105.2536 124.21) (end 104.14 125.3236) (width 0.25) (layer F.Cu) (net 22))
 (segment (start 104.14 125.3236) (end 104.14 125.476) (width 0.25) (layer F.Cu) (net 22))
 (segment (start 107.95 115.57) (end 107.95 124.0536) (width 0.25) (layer F.Cu) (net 21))
 (segment (start 107.95 124.0536) (end 106.68 125.3236) (width 0.25) (layer F.Cu) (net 21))
 (segment (start 106.68 125.3236) (end 106.68 125.476) (width 0.25) (layer F.Cu) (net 21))
 (segment (start 109.22 125.476) (end 109.22 124.21) (width 0.25) (layer F.Cu) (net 20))
 (segment (start 109.22 124.21) (end 109.22 116.205) (width 0.25) (layer F.Cu) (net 20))
 (segment (start 111.76 124.21) (end 111.76 125.476) (width 0.25) (layer F.Cu) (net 19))
 (segment (start 110.49 115.57) (end 110.49 122.94) (width 0.25) (layer F.Cu) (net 19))
 (segment (start 110.49 122.94) (end 111.76 124.21) (width 0.25) (layer F.Cu) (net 19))
 (segment (start 114.3 125.476) (end 114.3 124.21) (width 0.25) (layer F.Cu) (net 18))
 (segment (start 114.3 124.21) (end 111.76 121.67) (width 0.25) (layer F.Cu) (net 18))
 (segment (start 111.76 121.67) (end 111.76 116.205) (width 0.25) (layer F.Cu) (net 18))
 (segment (start 116.84 125.3236) (end 116.84 125.476) (width 0.25) (layer F.Cu) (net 17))
 (segment (start 113.03 115.57) (end 113.03 121.5136) (width 0.25) (layer F.Cu) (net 17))
 (segment (start 113.03 121.5136) (end 116.84 125.3236) (width 0.25) (layer F.Cu) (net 17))
 (segment (start 114.3 120.2436) (end 114.3 116.205) (width 0.25) (layer F.Cu) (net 16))
 (segment (start 119.38 125.476) (end 119.38 125.3236) (width 0.25) (layer F.Cu) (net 16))
 (segment (start 119.38 125.3236) (end 114.3 120.2436) (width 0.25) (layer F.Cu) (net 16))
 (segment (start 115.57 115.57) (end 115.57 118.9736) (width 0.25) (layer F.Cu) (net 15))
 (segment (start 115.57 118.9736) (end 121.92 125.3236) (width 0.25) (layer F.Cu) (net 15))
 (segment (start 121.92 125.3236) (end 121.92 125.476) (width 0.25) (layer F.Cu) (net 15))
 (segment (start 116.84 116.205) (end 116.84 117.856) (width 0.25) (layer F.Cu) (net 14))
 (segment (start 116.84 117.856) (end 123.194 124.21) (width 0.25) (layer F.Cu) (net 14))
 (segment (start 123.194 124.21) (end 123.3464 124.21) (width 0.25) (layer F.Cu) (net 14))
 (segment (start 123.3464 124.21) (end 124.46 125.3236) (width 0.25) (layer F.Cu) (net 14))
 (segment (start 124.46 125.3236) (end 124.46 125.476) (width 0.25) (layer F.Cu) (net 14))
 (segment (start 119.38 114.554) (end 119.126 114.3) (width 0.25) (layer F.Cu) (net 27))
 (segment (start 119.38 118.106) (end 119.38 114.554) (width 0.25) (layer F.Cu) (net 27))
 (segment (start 123.194 121.92) (end 119.38 118.106) (width 0.25) (layer F.Cu) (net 27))
 (segment (start 124.46 121.92) (end 123.194 121.92) (width 0.25) (layer F.Cu) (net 27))
 (segment (start 119.126 114.3) (end 118.745 114.3) (width 0.25) (layer F.Cu) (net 27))
 (segment (start 120.142 113.03) (end 120.904 113.792) (width 0.25) (layer F.Cu) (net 28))
 (segment (start 118.11 113.03) (end 120.142 113.03) (width 0.25) (layer F.Cu) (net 28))
 (segment (start 120.904 113.792) (end 120.904 115.9764) (width 0.25) (layer F.Cu) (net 28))
 (segment (start 120.904 115.9764) (end 124.3076 119.38) (width 0.25) (layer F.Cu) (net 28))
 (segment (start 124.3076 119.38) (end 124.46 119.38) (width 0.25) (layer F.Cu) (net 28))
 (segment (start 121.92 113.03) (end 121.92 114.4524) (width 0.25) (layer F.Cu) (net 29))
 (segment (start 118.745 111.76) (end 120.65 111.76) (width 0.25) (layer F.Cu) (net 29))
 (segment (start 120.65 111.76) (end 121.92 113.03) (width 0.25) (layer F.Cu) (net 29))
 (segment (start 121.92 114.4524) (end 124.3076 116.84) (width 0.25) (layer F.Cu) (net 29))
 (segment (start 124.3076 116.84) (end 124.46 116.84) (width 0.25) (layer F.Cu) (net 29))
 (segment (start 118.745 110.49) (end 118.872 110.49) (width 0.25) (layer F.Cu) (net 30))
 (segment (start 118.872 110.49) (end 121.158 110.49) (width 0.25) (layer F.Cu) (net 30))
 (segment (start 122.682 112.014) (end 122.682 112.6744) (width 0.25) (layer F.Cu) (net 30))
 (segment (start 121.158 110.49) (end 122.682 112.014) (width 0.25) (layer F.Cu) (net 30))
 (segment (start 122.682 112.6744) (end 124.3076 114.3) (width 0.25) (layer F.Cu) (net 30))
 (segment (start 124.3076 114.3) (end 124.46 114.3) (width 0.25) (layer F.Cu) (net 30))
 (segment (start 118.745 109.22) (end 121.666 109.22) (width 0.25) (layer F.Cu) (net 31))
 (segment (start 124.46 111.76) (end 124.3076 111.76) (width 0.25) (layer F.Cu) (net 31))
 (segment (start 124.3076 111.76) (end 121.7676 109.22) (width 0.25) (layer F.Cu) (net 31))
 (segment (start 121.7676 109.22) (end 121.666 109.22) (width 0.25) (layer F.Cu) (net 31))
 (segment (start 118.11 107.95) (end 123.0376 107.95) (width 0.25) (layer F.Cu) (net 32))
 (segment (start 123.0376 107.95) (end 124.3076 109.22) (width 0.25) (layer F.Cu) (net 32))
 (segment (start 124.3076 109.22) (end 124.46 109.22) (width 0.25) (layer F.Cu) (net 32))
 (segment (start 118.745 106.68) (end 124.46 106.68) (width 0.25) (layer F.Cu) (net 33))
 (segment (start 118.11 105.41) (end 123.0376 105.41) (width 0.25) (layer F.Cu) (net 34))
 (segment (start 123.0376 105.41) (end 124.3076 104.14) (width 0.25) (layer F.Cu) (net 34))
 (segment (start 124.3076 104.14) (end 124.46 104.14) (width 0.25) (layer F.Cu) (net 34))
 (segment (start 118.745 104.14) (end 121.7676 104.14) (width 0.25) (layer F.Cu) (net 35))
 (segment (start 121.7676 104.14) (end 124.3076 101.6) (width 0.25) (layer F.Cu) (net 35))
 (segment (start 124.3076 101.6) (end 124.46 101.6) (width 0.25) (layer F.Cu) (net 35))
 (segment (start 118.745 102.87) (end 119.126 102.87) (width 0.25) (layer F.Cu) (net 36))
 (segment (start 119.126 102.87) (end 121.158 102.87) (width 0.25) (layer F.Cu) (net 36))
 (segment (start 122.428 100.9396) (end 124.3076 99.06) (width 0.25) (layer F.Cu) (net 36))
 (segment (start 121.158 102.87) (end 122.428 101.6) (width 0.25) (layer F.Cu) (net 36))
 (segment (start 122.428 101.6) (end 122.428 100.9396) (width 0.25) (layer F.Cu) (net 36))
 (segment (start 124.3076 99.06) (end 124.46 99.06) (width 0.25) (layer F.Cu) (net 36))
 (segment (start 121.666 100.33) (end 121.666 99.1616) (width 0.25) (layer F.Cu) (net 37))
 (segment (start 118.745 101.6) (end 120.396 101.6) (width 0.25) (layer F.Cu) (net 37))
 (segment (start 120.396 101.6) (end 121.666 100.33) (width 0.25) (layer F.Cu) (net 37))
 (segment (start 121.666 99.1616) (end 124.3076 96.52) (width 0.25) (layer F.Cu) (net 37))
 (segment (start 124.3076 96.52) (end 124.46 96.52) (width 0.25) (layer F.Cu) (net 37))
 (segment (start 120.011 100.33) (end 120.65 99.691) (width 0.25) (layer F.Cu) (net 38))
 (segment (start 118.11 100.33) (end 120.011 100.33) (width 0.25) (layer F.Cu) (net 38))
 (segment (start 120.65 99.691) (end 120.65 97.536) (width 0.25) (layer F.Cu) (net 38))
 (segment (start 120.65 97.536) (end 120.7516 97.536) (width 0.25) (layer F.Cu) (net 38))
 (segment (start 120.7516 97.536) (end 124.3076 93.98) (width 0.25) (layer F.Cu) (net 38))
 (segment (start 124.3076 93.98) (end 124.46 93.98) (width 0.25) (layer F.Cu) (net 38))
 (segment (start 118.745 99.06) (end 119.38 98.425) (width 0.25) (layer F.Cu) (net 39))
 (segment (start 119.38 98.425) (end 119.38 95.504) (width 0.25) (layer F.Cu) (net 39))
 (segment (start 119.38 95.504) (end 123.444 91.44) (width 0.25) (layer F.Cu) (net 39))
 (segment (start 123.444 91.44) (end 124.46 91.44) (width 0.25) (layer F.Cu) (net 39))
 (segment (start 119.38 99.06) (end 119.38 95.504) (width 0.25) (layer F.Cu) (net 39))
 (segment (start 124.46 88.138) (end 116.84 95.758) (width 0.25) (layer F.Cu) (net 52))
 (segment (start 116.84 95.758) (end 116.84 97.155) (width 0.25) (layer F.Cu) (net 52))
 (segment (start 124.46 87.884) (end 124.46 88.138) (width 0.25) (layer F.Cu) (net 52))
 (segment (start 115.57 97.79) (end 115.57 95.504) (width 0.25) (layer F.Cu) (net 51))
 (segment (start 115.57 95.504) (end 121.92 89.154) (width 0.25) (layer F.Cu) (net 51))
 (segment (start 121.92 89.154) (end 121.92 87.884) (width 0.25) (layer F.Cu) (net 51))
 (segment (start 114.3 94.742) (end 119.38 89.662) (width 0.25) (layer F.Cu) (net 50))
 (segment (start 119.38 89.662) (end 119.38 87.884) (width 0.25) (layer F.Cu) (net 50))
 (segment (start 114.3 97.155) (end 114.3 94.742) (width 0.25) (layer F.Cu) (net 50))
 (segment (start 113.03 97.79) (end 113.03 93.218) (width 0.25) (layer F.Cu) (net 49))
 (segment (start 116.84 89.408) (end 116.84 87.884) (width 0.25) (layer F.Cu) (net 49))
 (segment (start 113.03 93.218) (end 116.84 89.408) (width 0.25) (layer F.Cu) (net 49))
 (segment (start 111.76 91.694) (end 114.3 89.154) (width 0.25) (layer F.Cu) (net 48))
 (segment (start 114.3 89.154) (end 114.3 87.884) (width 0.25) (layer F.Cu) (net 48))
 (segment (start 111.76 97.155) (end 111.76 91.694) (width 0.25) (layer F.Cu) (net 48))
 (segment (start 110.49 97.79) (end 110.49 90.678) (width 0.25) (layer F.Cu) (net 47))
 (segment (start 110.49 90.678) (end 111.76 89.408) (width 0.25) (layer F.Cu) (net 47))
 (segment (start 111.76 89.408) (end 111.76 87.884) (width 0.25) (layer F.Cu) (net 47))
 (segment (start 109.22 87.884) (end 109.22 97.155) (width 0.25) (layer F.Cu) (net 46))
 (segment (start 107.95 90.424) (end 106.68 89.154) (width 0.25) (layer F.Cu) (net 45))
 (segment (start 107.95 97.79) (end 107.95 90.424) (width 0.25) (layer F.Cu) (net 45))
 (segment (start 106.68 89.154) (end 106.68 87.884) (width 0.25) (layer F.Cu) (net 45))
 (segment (start 106.68 91.948) (end 104.14 89.408) (width 0.25) (layer F.Cu) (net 44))
 (segment (start 104.14 89.408) (end 104.14 87.884) (width 0.25) (layer F.Cu) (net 44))
 (segment (start 106.68 97.155) (end 106.68 91.948) (width 0.25) (layer F.Cu) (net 44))
 (segment (start 101.6 89.408) (end 101.6 87.884) (width 0.25) (layer F.Cu) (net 43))
 (segment (start 105.41 97.79) (end 105.41 93.218) (width 0.25) (layer F.Cu) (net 43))
 (segment (start 105.41 93.218) (end 101.6 89.408) (width 0.25) (layer F.Cu) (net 43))
 (segment (start 104.14 94.742) (end 99.06 89.662) (width 0.25) (layer F.Cu) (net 42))
 (segment (start 99.06 89.662) (end 99.06 87.884) (width 0.25) (layer F.Cu) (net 42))
 (segment (start 104.14 97.155) (end 104.14 94.742) (width 0.25) (layer F.Cu) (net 42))
 (segment (start 102.87 97.282) (end 102.87 95.25) (width 0.25) (layer F.Cu) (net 41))
 (segment (start 102.87 95.25) (end 96.52 88.9) (width 0.25) (layer F.Cu) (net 41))
 (segment (start 96.52 88.9) (end 96.52 87.884) (width 0.25) (layer F.Cu) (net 41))
 (segment (start 93.98 87.884) (end 93.98 88.0364) (width 0.25) (layer F.Cu) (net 40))
 (segment (start 101.6 95.889) (end 101.6 97.155) (width 0.25) (layer F.Cu) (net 40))
 (segment (start 93.98 88.0364) (end 101.6 95.6564) (width 0.25) (layer F.Cu) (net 40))
 (segment (start 101.6 95.6564) (end 101.6 95.889) (width 0.25) (layer F.Cu) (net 40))
 (segment (start 95.246 91.44) (end 95.5 91.694) (width 0.25) (layer F.Cu) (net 1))
 (segment (start 99.06 95.254) (end 95.5 91.694) (width 0.25) (layer F.Cu) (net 1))
 (segment (start 99.06 99.06) (end 99.06 95.254) (width 0.25) (layer F.Cu) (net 1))
 (segment (start 93.98 91.44) (end 95.246 91.44) (width 0.25) (layer F.Cu) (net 1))
 (segment (start 100.33 100.33) (end 98.298 100.33) (width 0.25) (layer F.Cu) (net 2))
 (segment (start 98.298 100.33) (end 97.79 99.822) (width 0.25) (layer F.Cu) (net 2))
 (segment (start 98.298 100.33) (end 99.695 100.33) (width 0.25) (layer F.Cu) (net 2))
 (segment (start 97.79 99.822) (end 97.79 96.524) (width 0.25) (layer F.Cu) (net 2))
 (segment (start 95.246 93.98) (end 97.79 96.524) (width 0.25) (layer F.Cu) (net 2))
 (segment (start 93.98 93.98) (end 95.246 93.98) (width 0.25) (layer F.Cu) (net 2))
 (segment (start 96.774 100.33) (end 98.044 101.6) (width 0.25) (layer F.Cu) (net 3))
 (segment (start 95.504 96.52) (end 96.774 97.79) (width 0.25) (layer F.Cu) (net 3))
 (segment (start 96.774 97.79) (end 96.774 100.33) (width 0.25) (layer F.Cu) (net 3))
 (segment (start 93.98 96.52) (end 95.504 96.52) (width 0.25) (layer F.Cu) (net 3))
 (segment (start 98.044 101.6) (end 99.695 101.6) (width 0.25) (layer F.Cu) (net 3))
 (segment (start 93.98 99.06) (end 94.1324 99.06) (width 0.25) (layer F.Cu) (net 4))
 (segment (start 97.9424 102.87) (end 100.33 102.87) (width 0.25) (layer F.Cu) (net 4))
 (segment (start 94.1324 99.06) (end 97.9424 102.87) (width 0.25) (layer F.Cu) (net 4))
 (segment (start 93.98 101.6) (end 95.246 101.6) (width 0.25) (layer F.Cu) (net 5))
 (segment (start 98.429 104.14) (end 99.695 104.14) (width 0.25) (layer F.Cu) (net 5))
 (segment (start 95.246 101.6) (end 97.786 104.14) (width 0.25) (layer F.Cu) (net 5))
 (segment (start 97.786 104.14) (end 98.429 104.14) (width 0.25) (layer F.Cu) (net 5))
 (segment (start 93.98 104.14) (end 95.246 104.14) (width 0.25) (layer F.Cu) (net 6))
 (segment (start 95.246 104.14) (end 96.516 105.41) (width 0.25) (layer F.Cu) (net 6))
 (segment (start 96.516 105.41) (end 100.33 105.41) (width 0.25) (layer F.Cu) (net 6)))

